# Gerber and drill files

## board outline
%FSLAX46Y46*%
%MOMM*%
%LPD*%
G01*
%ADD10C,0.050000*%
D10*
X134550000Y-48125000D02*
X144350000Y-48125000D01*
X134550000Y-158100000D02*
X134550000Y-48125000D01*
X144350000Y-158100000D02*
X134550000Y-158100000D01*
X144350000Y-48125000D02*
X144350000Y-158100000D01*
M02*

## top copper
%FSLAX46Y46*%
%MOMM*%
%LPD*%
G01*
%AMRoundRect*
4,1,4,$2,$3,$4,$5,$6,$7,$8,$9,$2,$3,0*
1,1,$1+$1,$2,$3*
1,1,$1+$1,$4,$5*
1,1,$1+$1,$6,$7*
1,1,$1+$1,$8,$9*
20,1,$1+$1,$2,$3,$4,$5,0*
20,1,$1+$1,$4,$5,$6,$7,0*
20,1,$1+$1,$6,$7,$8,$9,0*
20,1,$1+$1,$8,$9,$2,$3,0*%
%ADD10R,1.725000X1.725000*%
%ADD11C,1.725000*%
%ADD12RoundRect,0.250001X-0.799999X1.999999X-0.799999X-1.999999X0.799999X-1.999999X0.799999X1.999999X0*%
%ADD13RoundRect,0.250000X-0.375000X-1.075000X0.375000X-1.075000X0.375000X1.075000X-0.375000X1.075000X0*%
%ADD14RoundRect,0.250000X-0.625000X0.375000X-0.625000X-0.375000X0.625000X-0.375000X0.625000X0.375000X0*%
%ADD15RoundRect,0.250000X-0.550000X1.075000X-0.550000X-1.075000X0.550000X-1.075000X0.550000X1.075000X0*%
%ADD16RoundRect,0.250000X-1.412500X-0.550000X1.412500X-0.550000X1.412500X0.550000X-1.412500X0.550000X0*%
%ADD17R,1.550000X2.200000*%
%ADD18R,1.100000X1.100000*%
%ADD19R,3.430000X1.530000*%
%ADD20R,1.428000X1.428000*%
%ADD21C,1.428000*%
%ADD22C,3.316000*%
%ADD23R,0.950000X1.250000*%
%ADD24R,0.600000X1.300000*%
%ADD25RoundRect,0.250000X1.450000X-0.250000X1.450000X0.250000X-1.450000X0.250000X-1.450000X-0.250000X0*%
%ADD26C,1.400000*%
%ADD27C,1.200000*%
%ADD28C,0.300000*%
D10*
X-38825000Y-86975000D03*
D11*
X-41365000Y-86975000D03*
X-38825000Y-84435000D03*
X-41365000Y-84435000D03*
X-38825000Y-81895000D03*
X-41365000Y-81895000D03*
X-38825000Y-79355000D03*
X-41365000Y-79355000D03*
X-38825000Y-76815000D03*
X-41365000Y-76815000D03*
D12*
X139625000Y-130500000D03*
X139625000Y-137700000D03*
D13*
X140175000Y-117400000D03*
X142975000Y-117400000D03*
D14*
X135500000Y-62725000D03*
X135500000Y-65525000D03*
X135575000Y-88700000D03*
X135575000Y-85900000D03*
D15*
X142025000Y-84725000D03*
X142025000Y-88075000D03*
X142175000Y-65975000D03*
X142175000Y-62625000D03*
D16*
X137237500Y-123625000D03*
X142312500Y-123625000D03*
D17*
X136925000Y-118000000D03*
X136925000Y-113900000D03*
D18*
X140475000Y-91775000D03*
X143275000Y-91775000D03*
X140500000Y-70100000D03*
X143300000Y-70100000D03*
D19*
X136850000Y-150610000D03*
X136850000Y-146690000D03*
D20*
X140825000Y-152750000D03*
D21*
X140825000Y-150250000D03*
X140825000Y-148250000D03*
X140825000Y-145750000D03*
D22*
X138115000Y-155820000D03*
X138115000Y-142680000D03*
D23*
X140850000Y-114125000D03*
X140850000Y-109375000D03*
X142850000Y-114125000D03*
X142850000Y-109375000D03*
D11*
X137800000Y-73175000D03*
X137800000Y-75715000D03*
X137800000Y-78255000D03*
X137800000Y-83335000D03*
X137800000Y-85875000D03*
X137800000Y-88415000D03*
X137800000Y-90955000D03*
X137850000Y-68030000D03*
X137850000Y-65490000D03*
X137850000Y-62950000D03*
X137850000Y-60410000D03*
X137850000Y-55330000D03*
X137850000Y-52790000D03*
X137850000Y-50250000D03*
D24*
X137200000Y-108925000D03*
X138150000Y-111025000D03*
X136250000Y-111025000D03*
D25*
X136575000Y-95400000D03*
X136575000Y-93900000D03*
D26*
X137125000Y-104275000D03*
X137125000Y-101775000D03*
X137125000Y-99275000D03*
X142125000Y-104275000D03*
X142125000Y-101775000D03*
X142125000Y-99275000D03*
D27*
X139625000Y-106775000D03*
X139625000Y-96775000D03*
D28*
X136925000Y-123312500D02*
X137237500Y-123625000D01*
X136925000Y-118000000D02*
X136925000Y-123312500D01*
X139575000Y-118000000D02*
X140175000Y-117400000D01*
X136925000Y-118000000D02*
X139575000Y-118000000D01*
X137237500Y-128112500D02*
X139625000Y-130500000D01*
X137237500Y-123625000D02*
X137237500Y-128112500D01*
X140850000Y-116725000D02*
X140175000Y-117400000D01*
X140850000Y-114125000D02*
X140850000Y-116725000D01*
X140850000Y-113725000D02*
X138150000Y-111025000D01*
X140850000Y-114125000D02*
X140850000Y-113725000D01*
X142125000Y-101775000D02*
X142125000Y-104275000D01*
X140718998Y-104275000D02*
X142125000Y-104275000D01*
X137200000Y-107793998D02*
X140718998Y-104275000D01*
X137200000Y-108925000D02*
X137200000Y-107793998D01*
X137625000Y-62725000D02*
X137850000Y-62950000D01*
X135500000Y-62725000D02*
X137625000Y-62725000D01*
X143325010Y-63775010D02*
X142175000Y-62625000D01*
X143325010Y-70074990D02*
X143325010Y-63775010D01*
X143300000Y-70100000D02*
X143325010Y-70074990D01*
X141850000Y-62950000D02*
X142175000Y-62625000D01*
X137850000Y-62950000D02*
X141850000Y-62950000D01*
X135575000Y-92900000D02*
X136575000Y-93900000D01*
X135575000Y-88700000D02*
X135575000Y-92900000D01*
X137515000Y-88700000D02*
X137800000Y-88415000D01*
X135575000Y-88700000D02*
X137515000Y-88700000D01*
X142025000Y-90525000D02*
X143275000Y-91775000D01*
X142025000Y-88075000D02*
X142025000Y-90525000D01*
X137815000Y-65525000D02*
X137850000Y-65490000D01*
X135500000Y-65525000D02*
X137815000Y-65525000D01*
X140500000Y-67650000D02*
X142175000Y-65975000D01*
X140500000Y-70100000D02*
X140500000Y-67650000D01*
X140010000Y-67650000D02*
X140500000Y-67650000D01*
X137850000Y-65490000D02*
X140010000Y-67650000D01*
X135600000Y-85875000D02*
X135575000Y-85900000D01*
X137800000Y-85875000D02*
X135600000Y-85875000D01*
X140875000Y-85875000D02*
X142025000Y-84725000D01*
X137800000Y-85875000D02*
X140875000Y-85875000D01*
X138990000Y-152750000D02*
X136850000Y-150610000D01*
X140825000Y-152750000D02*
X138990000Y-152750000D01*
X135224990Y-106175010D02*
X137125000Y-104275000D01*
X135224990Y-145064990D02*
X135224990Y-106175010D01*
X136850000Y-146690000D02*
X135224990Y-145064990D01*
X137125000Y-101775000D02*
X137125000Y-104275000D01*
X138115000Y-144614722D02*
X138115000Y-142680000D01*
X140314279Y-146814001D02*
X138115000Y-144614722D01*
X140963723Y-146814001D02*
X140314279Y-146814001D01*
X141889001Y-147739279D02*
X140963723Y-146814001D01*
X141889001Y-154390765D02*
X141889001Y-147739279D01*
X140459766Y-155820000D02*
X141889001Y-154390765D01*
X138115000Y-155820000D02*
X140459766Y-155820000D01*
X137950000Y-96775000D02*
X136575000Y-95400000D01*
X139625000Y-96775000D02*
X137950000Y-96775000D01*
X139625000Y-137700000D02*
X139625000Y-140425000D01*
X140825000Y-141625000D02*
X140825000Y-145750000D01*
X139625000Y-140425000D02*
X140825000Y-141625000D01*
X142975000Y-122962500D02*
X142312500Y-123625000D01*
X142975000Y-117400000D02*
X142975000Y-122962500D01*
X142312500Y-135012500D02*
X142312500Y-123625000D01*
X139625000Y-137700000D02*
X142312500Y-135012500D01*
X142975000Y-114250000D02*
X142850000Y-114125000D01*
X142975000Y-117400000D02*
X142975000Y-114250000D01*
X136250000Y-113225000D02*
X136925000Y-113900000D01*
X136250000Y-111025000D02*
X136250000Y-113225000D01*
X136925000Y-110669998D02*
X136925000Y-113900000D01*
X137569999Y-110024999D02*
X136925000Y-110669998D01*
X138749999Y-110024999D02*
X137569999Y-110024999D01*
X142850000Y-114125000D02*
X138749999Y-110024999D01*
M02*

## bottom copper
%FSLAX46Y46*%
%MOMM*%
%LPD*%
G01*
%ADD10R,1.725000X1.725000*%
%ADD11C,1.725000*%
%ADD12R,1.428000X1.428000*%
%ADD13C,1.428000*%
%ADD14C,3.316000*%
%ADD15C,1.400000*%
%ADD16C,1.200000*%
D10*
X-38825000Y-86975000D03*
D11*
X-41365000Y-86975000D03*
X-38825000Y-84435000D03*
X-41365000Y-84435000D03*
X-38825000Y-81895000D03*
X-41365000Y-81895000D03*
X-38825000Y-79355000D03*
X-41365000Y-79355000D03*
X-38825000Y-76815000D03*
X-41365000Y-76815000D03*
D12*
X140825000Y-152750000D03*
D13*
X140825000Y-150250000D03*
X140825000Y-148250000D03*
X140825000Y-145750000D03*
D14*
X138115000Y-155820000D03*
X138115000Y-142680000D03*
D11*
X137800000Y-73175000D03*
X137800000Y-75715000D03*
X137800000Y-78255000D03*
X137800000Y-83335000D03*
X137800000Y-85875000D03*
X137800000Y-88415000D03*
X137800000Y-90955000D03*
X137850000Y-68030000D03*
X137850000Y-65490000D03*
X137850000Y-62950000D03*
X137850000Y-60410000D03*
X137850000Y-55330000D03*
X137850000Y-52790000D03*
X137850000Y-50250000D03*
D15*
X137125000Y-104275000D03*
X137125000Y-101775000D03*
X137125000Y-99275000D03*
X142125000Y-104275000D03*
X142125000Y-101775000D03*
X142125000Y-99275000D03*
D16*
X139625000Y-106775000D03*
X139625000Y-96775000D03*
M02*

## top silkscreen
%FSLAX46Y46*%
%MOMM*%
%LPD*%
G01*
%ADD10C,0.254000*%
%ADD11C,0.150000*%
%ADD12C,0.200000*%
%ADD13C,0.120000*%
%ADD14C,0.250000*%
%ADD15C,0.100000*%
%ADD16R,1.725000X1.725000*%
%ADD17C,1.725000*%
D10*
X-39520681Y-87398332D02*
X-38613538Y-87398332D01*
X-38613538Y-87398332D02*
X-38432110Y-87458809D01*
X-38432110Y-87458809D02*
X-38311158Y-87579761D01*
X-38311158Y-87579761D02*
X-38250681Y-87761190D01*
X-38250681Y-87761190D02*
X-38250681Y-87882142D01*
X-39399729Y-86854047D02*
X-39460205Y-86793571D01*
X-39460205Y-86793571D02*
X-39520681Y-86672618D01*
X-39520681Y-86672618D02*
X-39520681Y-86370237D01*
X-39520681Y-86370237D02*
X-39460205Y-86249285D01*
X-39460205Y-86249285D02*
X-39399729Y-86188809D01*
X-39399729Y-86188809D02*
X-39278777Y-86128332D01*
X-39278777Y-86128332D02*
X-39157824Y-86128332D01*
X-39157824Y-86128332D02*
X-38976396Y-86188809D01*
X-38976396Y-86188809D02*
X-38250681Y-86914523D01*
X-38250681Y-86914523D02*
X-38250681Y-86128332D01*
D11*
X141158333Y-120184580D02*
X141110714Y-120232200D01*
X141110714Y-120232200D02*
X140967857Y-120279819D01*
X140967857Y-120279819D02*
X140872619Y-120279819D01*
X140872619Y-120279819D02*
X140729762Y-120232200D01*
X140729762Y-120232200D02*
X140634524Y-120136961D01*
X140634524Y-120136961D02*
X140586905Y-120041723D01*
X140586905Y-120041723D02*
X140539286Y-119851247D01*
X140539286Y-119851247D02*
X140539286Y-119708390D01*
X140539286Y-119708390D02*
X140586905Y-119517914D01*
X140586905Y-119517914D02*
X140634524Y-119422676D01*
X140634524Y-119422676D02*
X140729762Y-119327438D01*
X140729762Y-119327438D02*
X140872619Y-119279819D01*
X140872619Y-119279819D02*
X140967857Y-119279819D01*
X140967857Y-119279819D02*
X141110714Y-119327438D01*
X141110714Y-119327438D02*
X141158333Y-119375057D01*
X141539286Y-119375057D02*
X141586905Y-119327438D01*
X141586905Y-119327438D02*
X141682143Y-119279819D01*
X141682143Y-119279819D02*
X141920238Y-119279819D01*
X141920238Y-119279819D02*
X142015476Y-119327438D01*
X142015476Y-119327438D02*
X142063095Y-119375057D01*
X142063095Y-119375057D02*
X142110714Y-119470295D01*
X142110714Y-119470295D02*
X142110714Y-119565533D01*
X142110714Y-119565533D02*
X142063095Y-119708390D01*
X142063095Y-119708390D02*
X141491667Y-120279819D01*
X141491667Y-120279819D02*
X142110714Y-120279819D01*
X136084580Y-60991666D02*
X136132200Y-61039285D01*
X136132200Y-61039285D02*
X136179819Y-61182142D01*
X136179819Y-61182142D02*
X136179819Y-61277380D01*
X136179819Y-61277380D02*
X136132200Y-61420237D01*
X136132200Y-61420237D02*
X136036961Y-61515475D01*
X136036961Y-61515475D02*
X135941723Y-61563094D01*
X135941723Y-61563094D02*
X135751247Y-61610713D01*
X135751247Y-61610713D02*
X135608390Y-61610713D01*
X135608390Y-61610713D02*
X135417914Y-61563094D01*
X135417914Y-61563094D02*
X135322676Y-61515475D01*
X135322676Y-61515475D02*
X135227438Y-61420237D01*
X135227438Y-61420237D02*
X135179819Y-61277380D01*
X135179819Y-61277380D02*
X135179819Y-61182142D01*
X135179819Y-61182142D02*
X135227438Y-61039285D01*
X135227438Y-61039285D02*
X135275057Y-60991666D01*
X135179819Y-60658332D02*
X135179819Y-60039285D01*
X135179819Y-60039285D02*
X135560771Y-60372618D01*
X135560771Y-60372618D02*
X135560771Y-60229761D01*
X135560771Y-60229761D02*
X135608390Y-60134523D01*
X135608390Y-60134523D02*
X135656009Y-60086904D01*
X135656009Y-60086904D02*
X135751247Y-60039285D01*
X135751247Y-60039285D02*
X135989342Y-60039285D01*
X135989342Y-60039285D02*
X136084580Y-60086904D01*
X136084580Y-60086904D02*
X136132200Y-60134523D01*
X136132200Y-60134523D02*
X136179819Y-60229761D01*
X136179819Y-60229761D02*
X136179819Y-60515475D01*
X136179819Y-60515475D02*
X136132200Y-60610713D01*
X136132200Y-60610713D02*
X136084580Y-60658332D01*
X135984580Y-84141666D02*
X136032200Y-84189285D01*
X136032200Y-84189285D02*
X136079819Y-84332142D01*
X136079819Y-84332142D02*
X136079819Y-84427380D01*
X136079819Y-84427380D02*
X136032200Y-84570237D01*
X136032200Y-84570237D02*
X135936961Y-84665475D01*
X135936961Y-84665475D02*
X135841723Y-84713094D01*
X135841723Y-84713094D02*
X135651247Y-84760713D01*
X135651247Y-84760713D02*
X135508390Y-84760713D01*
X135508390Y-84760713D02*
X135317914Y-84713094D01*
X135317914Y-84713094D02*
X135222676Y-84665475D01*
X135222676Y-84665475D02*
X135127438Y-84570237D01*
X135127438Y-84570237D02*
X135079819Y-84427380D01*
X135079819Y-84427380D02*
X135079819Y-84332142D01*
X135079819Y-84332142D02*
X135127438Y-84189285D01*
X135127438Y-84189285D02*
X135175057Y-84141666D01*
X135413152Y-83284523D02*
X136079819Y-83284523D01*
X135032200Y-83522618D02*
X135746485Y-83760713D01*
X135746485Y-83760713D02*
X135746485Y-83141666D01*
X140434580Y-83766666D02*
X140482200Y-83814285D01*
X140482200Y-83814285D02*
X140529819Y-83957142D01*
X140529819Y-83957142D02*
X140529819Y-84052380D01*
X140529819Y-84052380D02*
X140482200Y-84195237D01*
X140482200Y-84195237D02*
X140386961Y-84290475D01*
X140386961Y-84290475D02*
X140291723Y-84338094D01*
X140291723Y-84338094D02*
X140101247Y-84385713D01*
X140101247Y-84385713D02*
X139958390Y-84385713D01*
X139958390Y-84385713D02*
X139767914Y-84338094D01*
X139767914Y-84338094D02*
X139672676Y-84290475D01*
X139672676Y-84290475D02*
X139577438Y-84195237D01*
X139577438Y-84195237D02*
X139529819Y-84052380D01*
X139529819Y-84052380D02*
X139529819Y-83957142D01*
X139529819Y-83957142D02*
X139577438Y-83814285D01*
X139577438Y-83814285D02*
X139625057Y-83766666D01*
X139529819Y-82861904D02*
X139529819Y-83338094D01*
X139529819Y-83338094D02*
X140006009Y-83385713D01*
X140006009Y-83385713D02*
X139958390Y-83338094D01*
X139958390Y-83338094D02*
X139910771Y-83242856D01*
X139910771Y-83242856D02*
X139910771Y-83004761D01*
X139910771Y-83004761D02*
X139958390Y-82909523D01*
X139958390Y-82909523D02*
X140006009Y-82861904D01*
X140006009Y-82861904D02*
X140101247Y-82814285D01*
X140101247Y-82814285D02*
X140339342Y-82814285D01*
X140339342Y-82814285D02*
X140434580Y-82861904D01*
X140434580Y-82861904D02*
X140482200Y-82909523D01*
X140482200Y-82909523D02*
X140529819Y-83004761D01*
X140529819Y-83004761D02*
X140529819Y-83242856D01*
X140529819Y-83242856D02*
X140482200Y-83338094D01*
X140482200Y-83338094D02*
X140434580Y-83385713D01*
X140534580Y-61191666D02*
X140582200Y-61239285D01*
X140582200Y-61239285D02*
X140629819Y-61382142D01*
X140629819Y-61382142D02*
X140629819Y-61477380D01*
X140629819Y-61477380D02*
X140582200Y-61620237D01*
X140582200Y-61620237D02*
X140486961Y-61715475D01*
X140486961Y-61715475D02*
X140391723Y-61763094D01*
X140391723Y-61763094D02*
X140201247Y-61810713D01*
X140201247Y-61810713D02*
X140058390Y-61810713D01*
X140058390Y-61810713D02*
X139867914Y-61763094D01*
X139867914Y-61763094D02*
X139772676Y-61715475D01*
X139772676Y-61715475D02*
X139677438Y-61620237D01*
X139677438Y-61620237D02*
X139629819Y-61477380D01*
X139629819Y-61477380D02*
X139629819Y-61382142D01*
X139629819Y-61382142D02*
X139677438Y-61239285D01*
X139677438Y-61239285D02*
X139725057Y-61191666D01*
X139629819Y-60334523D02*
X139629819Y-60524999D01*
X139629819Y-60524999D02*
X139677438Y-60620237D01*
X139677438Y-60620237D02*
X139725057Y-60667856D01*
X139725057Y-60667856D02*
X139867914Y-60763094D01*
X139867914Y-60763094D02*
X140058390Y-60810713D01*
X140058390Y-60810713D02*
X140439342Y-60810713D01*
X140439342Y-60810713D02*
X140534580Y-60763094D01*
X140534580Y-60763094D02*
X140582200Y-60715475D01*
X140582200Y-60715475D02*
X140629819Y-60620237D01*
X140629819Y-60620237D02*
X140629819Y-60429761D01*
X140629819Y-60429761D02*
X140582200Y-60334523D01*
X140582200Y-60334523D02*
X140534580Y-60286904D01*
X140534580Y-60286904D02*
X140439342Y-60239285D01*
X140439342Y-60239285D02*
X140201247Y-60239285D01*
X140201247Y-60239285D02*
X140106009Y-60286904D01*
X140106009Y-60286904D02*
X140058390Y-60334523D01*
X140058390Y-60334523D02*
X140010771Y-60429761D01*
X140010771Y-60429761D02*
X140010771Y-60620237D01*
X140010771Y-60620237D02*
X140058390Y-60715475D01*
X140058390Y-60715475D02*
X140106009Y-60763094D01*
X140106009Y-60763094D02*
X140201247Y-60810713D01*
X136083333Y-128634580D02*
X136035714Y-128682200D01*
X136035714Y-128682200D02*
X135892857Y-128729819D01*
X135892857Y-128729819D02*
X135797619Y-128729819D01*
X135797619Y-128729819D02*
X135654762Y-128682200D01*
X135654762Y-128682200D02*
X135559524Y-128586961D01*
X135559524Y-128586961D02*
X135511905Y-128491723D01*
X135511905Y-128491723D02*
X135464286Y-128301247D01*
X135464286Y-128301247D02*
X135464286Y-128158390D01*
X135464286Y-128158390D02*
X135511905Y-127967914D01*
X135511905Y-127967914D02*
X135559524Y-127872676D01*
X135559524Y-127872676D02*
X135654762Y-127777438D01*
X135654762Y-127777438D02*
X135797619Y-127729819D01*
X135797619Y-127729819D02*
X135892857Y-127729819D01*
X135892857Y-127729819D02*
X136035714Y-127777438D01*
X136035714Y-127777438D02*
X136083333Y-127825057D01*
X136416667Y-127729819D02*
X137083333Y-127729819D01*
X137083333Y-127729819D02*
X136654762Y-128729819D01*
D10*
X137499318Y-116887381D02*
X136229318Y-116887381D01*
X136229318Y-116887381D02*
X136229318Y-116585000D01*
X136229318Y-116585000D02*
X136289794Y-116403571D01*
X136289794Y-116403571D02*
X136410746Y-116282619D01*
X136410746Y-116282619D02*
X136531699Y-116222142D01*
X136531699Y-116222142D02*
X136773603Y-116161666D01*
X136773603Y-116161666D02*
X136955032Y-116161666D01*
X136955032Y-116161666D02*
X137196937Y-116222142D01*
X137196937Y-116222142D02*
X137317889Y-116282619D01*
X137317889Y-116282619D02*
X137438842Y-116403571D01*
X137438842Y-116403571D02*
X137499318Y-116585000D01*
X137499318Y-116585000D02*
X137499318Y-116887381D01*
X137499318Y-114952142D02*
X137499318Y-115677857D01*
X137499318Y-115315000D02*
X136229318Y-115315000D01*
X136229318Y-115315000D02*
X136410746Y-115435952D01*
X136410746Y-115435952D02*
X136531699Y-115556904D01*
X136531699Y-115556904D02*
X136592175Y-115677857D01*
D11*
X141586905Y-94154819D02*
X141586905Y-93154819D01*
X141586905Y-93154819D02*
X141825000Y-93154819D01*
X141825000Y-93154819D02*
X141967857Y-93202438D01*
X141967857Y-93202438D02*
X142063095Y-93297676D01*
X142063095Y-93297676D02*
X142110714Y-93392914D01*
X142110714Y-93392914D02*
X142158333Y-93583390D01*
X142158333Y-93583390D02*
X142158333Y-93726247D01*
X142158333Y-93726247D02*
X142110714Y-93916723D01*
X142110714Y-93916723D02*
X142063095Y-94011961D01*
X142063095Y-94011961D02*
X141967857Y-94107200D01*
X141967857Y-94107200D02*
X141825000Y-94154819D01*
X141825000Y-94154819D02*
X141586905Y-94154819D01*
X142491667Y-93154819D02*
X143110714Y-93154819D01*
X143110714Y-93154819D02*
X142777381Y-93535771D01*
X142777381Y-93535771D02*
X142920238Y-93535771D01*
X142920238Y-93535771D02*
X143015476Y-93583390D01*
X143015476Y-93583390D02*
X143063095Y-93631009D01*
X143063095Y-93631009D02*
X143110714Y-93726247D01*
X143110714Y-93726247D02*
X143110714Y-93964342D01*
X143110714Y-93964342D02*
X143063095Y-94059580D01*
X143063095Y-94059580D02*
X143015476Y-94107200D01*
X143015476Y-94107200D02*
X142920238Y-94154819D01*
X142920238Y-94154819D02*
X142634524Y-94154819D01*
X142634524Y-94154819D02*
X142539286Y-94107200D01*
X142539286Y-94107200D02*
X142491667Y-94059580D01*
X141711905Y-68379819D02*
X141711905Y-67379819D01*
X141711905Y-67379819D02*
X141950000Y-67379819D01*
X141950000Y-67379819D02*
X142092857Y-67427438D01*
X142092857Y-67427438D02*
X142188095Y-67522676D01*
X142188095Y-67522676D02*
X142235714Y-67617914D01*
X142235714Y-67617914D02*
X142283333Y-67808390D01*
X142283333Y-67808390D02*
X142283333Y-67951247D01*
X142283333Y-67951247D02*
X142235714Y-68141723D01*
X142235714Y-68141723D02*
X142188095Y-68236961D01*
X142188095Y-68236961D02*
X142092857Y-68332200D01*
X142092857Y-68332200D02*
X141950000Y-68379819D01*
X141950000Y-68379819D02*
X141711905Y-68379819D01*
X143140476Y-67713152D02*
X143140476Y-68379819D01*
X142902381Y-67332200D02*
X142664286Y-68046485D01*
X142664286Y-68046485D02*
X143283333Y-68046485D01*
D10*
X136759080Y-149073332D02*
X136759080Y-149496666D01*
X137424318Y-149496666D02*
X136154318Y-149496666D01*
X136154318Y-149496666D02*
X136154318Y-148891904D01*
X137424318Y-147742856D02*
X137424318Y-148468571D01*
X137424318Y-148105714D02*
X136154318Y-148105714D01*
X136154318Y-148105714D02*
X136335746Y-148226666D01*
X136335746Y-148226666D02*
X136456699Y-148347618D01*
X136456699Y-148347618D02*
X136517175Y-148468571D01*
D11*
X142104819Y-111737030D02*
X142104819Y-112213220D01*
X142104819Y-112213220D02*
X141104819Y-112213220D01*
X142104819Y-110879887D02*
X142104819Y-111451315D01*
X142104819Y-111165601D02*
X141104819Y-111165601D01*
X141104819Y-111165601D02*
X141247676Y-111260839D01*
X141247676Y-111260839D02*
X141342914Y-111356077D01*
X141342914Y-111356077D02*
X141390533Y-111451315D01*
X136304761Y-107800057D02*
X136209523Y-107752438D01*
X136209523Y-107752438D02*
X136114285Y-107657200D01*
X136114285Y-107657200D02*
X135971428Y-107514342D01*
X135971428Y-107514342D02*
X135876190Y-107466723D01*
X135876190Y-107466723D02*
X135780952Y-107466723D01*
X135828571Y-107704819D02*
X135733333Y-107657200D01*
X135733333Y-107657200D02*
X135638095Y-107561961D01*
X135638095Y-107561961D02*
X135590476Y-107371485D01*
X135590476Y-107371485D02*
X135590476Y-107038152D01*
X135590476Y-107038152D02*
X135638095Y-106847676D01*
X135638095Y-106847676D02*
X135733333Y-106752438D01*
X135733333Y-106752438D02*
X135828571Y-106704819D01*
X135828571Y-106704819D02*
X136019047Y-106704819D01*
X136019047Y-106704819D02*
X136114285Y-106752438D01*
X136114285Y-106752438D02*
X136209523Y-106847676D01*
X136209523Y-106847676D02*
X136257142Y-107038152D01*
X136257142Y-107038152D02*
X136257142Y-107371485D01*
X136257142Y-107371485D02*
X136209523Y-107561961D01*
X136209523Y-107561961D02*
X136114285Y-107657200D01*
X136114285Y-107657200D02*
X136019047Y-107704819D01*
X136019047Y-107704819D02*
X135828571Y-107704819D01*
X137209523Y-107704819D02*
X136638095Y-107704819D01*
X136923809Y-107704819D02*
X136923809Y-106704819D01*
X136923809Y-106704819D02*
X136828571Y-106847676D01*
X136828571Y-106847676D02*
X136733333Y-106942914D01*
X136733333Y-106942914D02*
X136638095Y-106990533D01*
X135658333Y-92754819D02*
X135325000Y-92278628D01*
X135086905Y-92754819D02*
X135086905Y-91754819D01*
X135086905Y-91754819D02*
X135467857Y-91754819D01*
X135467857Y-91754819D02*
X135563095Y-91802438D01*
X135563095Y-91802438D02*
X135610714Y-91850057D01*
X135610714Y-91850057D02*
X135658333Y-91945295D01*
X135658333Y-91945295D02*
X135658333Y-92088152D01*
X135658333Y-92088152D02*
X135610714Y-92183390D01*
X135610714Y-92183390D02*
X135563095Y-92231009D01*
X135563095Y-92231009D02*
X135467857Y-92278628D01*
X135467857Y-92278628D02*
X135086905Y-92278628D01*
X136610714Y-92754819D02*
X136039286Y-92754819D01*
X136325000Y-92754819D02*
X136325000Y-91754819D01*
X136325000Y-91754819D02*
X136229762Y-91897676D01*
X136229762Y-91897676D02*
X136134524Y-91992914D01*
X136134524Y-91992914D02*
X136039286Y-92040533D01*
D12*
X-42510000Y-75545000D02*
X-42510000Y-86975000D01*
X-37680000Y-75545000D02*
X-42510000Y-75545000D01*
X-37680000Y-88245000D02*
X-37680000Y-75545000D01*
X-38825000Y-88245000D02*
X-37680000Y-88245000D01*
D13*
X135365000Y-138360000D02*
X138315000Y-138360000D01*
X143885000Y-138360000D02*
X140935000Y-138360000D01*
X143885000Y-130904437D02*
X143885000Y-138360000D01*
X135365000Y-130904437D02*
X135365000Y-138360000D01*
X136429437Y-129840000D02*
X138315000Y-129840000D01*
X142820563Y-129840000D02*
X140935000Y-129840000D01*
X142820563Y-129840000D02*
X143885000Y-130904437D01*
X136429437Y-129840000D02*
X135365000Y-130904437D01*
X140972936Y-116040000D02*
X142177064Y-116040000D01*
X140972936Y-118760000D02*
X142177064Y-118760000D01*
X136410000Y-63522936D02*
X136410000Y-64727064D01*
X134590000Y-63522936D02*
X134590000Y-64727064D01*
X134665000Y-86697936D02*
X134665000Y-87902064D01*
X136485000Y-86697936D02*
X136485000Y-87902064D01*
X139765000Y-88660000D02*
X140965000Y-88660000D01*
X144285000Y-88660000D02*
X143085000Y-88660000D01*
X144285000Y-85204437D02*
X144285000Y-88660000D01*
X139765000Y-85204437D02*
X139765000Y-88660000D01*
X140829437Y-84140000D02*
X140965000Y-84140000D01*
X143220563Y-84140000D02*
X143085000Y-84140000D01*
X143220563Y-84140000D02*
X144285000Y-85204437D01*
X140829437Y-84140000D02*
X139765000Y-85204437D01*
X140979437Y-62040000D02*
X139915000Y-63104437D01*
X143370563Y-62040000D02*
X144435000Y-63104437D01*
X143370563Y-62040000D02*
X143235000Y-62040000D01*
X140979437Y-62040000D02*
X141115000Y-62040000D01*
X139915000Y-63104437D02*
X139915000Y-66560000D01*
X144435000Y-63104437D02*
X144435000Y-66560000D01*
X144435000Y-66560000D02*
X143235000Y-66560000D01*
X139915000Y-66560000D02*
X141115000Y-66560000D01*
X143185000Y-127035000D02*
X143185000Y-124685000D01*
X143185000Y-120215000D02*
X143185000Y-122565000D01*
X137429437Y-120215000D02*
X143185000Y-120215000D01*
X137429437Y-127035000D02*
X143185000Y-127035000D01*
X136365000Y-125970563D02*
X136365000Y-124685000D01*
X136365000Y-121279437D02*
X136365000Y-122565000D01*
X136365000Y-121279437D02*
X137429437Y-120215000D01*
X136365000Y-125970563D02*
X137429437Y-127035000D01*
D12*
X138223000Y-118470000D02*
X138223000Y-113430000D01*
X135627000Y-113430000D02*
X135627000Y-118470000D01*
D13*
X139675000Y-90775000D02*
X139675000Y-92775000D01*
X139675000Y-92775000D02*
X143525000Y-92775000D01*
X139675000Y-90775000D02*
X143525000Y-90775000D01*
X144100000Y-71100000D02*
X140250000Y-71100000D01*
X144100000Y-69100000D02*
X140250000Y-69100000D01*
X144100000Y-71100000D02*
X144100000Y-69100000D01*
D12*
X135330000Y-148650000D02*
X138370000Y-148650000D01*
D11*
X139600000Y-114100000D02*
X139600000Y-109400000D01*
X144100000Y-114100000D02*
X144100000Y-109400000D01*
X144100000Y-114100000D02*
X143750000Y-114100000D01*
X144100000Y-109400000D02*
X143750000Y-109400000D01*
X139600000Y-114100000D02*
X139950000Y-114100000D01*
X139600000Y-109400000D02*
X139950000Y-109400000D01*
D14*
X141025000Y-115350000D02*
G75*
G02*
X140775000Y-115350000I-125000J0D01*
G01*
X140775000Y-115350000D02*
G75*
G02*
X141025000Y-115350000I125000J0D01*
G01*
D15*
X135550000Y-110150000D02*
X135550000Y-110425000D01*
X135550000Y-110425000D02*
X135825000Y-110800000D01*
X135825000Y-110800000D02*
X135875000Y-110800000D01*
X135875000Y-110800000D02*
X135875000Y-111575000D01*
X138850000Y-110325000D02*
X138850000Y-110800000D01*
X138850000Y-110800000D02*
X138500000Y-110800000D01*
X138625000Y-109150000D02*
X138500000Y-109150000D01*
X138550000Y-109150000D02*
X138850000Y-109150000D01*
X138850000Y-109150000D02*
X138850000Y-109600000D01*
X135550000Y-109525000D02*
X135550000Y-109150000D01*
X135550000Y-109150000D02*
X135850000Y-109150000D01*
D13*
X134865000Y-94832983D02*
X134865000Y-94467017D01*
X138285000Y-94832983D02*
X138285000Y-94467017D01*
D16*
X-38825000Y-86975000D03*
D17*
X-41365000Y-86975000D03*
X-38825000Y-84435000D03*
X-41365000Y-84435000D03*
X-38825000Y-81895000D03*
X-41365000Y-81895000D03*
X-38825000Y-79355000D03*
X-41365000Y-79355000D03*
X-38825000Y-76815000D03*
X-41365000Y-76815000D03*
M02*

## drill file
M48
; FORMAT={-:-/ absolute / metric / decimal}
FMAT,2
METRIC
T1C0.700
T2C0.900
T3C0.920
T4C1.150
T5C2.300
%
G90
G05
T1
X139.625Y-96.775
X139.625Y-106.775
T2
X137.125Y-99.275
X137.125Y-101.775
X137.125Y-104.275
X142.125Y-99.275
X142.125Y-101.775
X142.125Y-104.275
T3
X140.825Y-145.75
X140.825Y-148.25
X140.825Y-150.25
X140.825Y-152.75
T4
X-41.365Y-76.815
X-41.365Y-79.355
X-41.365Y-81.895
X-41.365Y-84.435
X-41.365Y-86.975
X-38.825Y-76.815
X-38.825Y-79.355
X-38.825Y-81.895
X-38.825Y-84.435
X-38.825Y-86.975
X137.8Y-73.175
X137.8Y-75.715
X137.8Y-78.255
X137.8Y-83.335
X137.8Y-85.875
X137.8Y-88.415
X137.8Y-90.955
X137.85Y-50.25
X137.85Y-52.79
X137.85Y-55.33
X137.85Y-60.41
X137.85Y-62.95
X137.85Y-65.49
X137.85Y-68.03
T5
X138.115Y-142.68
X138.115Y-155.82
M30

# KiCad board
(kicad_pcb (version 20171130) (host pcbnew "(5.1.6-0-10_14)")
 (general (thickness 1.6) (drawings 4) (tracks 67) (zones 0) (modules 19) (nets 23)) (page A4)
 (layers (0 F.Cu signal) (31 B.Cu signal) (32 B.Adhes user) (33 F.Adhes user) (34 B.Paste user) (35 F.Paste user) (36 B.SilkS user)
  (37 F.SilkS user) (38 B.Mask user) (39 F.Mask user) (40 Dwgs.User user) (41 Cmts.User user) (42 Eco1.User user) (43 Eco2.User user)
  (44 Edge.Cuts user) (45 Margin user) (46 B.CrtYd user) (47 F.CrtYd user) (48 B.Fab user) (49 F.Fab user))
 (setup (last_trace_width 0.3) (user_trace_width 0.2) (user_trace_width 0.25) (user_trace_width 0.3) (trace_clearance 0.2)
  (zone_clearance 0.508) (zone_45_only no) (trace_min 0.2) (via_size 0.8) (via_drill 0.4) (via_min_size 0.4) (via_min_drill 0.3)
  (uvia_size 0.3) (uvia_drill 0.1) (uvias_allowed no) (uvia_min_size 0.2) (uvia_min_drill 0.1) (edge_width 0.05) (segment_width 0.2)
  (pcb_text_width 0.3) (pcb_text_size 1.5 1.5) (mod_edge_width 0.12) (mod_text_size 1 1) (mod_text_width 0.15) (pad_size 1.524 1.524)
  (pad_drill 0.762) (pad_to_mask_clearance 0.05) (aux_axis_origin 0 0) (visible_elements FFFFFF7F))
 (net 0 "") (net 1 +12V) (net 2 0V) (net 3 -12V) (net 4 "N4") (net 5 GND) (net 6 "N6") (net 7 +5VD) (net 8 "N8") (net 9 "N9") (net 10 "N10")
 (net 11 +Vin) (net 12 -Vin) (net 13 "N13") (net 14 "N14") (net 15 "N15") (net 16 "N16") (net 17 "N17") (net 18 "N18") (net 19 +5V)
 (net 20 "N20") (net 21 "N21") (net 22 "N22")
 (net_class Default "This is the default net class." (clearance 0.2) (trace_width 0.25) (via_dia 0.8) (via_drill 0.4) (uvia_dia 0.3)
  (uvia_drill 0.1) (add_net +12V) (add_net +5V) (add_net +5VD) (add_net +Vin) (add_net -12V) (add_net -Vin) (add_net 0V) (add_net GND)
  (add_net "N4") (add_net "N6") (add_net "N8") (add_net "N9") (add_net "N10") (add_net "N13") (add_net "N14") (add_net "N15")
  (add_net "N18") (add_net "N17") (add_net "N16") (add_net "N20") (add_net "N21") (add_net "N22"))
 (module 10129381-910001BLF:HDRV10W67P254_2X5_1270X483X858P (layer F.Cu) (at -38.825 86.975 90)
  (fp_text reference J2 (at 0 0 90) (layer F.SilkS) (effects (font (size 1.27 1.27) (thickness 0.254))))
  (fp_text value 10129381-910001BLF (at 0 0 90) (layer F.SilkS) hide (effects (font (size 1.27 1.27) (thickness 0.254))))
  (fp_line (start 11.43 -3.685) (end 0 -3.685) (layer F.SilkS) (width 0.2))
  (fp_line (start 11.43 1.145) (end 11.43 -3.685) (layer F.SilkS) (width 0.2))
  (fp_line (start -1.27 1.145) (end 11.43 1.145) (layer F.SilkS) (width 0.2))
  (fp_line (start -1.27 0) (end -1.27 1.145) (layer F.SilkS) (width 0.2))
  (pad 1 thru_hole rect (at 0 0 180) (size 1.725 1.725) (drill 1.15) (layers *.Cu *.Mask F.SilkS) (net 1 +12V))
  (pad 2 thru_hole circle (at 0 -2.54 180) (size 1.725 1.725) (drill 1.15) (layers *.Cu *.Mask F.SilkS) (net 1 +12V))
  (pad 3 thru_hole circle (at 2.54 0 180) (size 1.725 1.725) (drill 1.15) (layers *.Cu *.Mask F.SilkS) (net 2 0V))
  (pad 4 thru_hole circle (at 2.54 -2.54 180) (size 1.725 1.725) (drill 1.15) (layers *.Cu *.Mask F.SilkS) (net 2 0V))
  (pad 5 thru_hole circle (at 5.08 0 180) (size 1.725 1.725) (drill 1.15) (layers *.Cu *.Mask F.SilkS) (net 2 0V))
  (pad 6 thru_hole circle (at 5.08 -2.54 180) (size 1.725 1.725) (drill 1.15) (layers *.Cu *.Mask F.SilkS) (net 2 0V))
  (pad 7 thru_hole circle (at 7.62 0 180) (size 1.725 1.725) (drill 1.15) (layers *.Cu *.Mask F.SilkS) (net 2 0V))
  (pad 8 thru_hole circle (at 7.62 -2.54 180) (size 1.725 1.725) (drill 1.15) (layers *.Cu *.Mask F.SilkS) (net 2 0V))
  (pad 9 thru_hole circle (at 10.16 0 180) (size 1.725 1.725) (drill 1.15) (layers *.Cu *.Mask F.SilkS) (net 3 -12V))
  (pad 10 thru_hole circle (at 10.16 -2.54 180) (size 1.725 1.725) (drill 1.15) (layers *.Cu *.Mask F.SilkS) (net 3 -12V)))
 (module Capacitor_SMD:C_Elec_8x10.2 (layer F.Cu) (at 139.625 134.1 270)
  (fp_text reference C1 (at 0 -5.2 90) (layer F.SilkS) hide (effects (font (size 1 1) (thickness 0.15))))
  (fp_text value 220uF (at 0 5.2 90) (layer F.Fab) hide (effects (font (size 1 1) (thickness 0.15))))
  (fp_line (start 4.26 4.26) (end 4.26 1.31) (layer F.SilkS) (width 0.12))
  (fp_line (start 4.26 -4.26) (end 4.26 -1.31) (layer F.SilkS) (width 0.12))
  (fp_line (start -3.195563 -4.26) (end 4.26 -4.26) (layer F.SilkS) (width 0.12))
  (fp_line (start -3.195563 4.26) (end 4.26 4.26) (layer F.SilkS) (width 0.12))
  (fp_line (start -4.26 3.195563) (end -4.26 1.31) (layer F.SilkS) (width 0.12))
  (fp_line (start -4.26 -3.195563) (end -4.26 -1.31) (layer F.SilkS) (width 0.12))
  (fp_line (start -4.26 -3.195563) (end -3.195563 -4.26) (layer F.SilkS) (width 0.12))
  (fp_line (start -4.26 3.195563) (end -3.195563 4.26) (layer F.SilkS) (width 0.12))
  (pad 1 smd roundrect (at -3.6 0 270) (size 4.5 2.1) (layers F.Cu F.Paste F.Mask) (roundrect_rratio 0.119048) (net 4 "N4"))
  (pad 2 smd roundrect (at 3.6 0 270) (size 4.5 2.1) (layers F.Cu F.Paste F.Mask) (roundrect_rratio 0.119048) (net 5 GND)))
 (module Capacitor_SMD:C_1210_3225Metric (layer F.Cu) (at 141.575 117.4)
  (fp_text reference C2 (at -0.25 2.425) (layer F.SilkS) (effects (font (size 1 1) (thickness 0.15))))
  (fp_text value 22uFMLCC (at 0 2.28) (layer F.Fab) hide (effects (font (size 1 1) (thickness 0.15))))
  (fp_line (start -0.602064 -1.36) (end 0.602064 -1.36) (layer F.SilkS) (width 0.12))
  (fp_line (start -0.602064 1.36) (end 0.602064 1.36) (layer F.SilkS) (width 0.12))
  (pad 1 smd roundrect (at -1.4 0) (size 1.25 2.65) (layers F.Cu F.Paste F.Mask) (roundrect_rratio 0.2) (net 4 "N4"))
  (pad 2 smd roundrect (at 1.4 0) (size 1.25 2.65) (layers F.Cu F.Paste F.Mask) (roundrect_rratio 0.2) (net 5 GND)))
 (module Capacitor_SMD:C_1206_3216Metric (layer F.Cu) (at 135.5 64.125 270)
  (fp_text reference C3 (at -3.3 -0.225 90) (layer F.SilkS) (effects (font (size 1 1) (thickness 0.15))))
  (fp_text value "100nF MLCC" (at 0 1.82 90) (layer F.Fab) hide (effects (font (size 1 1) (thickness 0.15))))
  (fp_line (start -0.602064 -0.91) (end 0.602064 -0.91) (layer F.SilkS) (width 0.12))
  (fp_line (start -0.602064 0.91) (end 0.602064 0.91) (layer F.SilkS) (width 0.12))
  (pad 1 smd roundrect (at -1.4 0 270) (size 1.25 1.75) (layers F.Cu F.Paste F.Mask) (roundrect_rratio 0.2) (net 2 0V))
  (pad 2 smd roundrect (at 1.4 0 270) (size 1.25 1.75) (layers F.Cu F.Paste F.Mask) (roundrect_rratio 0.2) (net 3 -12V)))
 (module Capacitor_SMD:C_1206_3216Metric (layer F.Cu) (at 135.575 87.3 270)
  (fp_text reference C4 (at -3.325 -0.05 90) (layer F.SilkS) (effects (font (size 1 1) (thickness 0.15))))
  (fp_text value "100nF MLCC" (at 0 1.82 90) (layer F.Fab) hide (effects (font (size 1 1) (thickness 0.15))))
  (fp_line (start -0.602064 0.91) (end 0.602064 0.91) (layer F.SilkS) (width 0.12))
  (fp_line (start -0.602064 -0.91) (end 0.602064 -0.91) (layer F.SilkS) (width 0.12))
  (pad 2 smd roundrect (at 1.4 0 270) (size 1.25 1.75) (layers F.Cu F.Paste F.Mask) (roundrect_rratio 0.2) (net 2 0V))
  (pad 1 smd roundrect (at -1.4 0 270) (size 1.25 1.75) (layers F.Cu F.Paste F.Mask) (roundrect_rratio 0.2) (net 1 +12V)))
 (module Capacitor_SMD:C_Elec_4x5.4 (layer F.Cu) (at 142.025 86.4 270)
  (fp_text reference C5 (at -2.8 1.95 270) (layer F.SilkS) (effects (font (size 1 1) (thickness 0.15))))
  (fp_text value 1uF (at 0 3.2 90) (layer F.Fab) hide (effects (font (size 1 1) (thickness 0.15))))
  (fp_line (start 2.26 2.26) (end 2.26 1.06) (layer F.SilkS) (width 0.12))
  (fp_line (start 2.26 -2.26) (end 2.26 -1.06) (layer F.SilkS) (width 0.12))
  (fp_line (start -1.195563 -2.26) (end 2.26 -2.26) (layer F.SilkS) (width 0.12))
  (fp_line (start -1.195563 2.26) (end 2.26 2.26) (layer F.SilkS) (width 0.12))
  (fp_line (start -2.26 1.195563) (end -2.26 1.06) (layer F.SilkS) (width 0.12))
  (fp_line (start -2.26 -1.195563) (end -2.26 -1.06) (layer F.SilkS) (width 0.12))
  (fp_line (start -2.26 -1.195563) (end -1.195563 -2.26) (layer F.SilkS) (width 0.12))
  (fp_line (start -2.26 1.195563) (end -1.195563 2.26) (layer F.SilkS) (width 0.12))
  (pad 1 smd roundrect (at -1.675 0 270) (size 2.65 1.6) (layers F.Cu F.Paste F.Mask) (roundrect_rratio 0.15625) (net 1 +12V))
  (pad 2 smd roundrect (at 1.675 0 270) (size 2.65 1.6) (layers F.Cu F.Paste F.Mask) (roundrect_rratio 0.15625) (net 2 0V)))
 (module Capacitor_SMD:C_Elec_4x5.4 (layer F.Cu) (at 142.175 64.3 270)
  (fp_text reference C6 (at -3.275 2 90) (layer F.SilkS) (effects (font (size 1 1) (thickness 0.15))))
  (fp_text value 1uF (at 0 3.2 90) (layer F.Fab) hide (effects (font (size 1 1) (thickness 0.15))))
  (fp_line (start -2.26 1.195563) (end -1.195563 2.26) (layer F.SilkS) (width 0.12))
  (fp_line (start -2.26 -1.195563) (end -1.195563 -2.26) (layer F.SilkS) (width 0.12))
  (fp_line (start -2.26 -1.195563) (end -2.26 -1.06) (layer F.SilkS) (width 0.12))
  (fp_line (start -2.26 1.195563) (end -2.26 1.06) (layer F.SilkS) (width 0.12))
  (fp_line (start -1.195563 2.26) (end 2.26 2.26) (layer F.SilkS) (width 0.12))
  (fp_line (start -1.195563 -2.26) (end 2.26 -2.26) (layer F.SilkS) (width 0.12))
  (fp_line (start 2.26 -2.26) (end 2.26 -1.06) (layer F.SilkS) (width 0.12))
  (fp_line (start 2.26 2.26) (end 2.26 1.06) (layer F.SilkS) (width 0.12))
  (pad 2 smd roundrect (at 1.675 0 270) (size 2.65 1.6) (layers F.Cu F.Paste F.Mask) (roundrect_rratio 0.15625) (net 3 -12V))
  (pad 1 smd roundrect (at -1.675 0 270) (size 2.65 1.6) (layers F.Cu F.Paste F.Mask) (roundrect_rratio 0.15625) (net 2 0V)))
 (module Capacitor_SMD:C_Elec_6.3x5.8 (layer F.Cu) (at 139.775 123.625)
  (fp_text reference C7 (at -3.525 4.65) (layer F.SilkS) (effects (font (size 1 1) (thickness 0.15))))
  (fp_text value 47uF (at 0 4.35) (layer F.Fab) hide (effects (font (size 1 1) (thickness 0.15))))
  (fp_line (start 3.41 3.41) (end 3.41 1.06) (layer F.SilkS) (width 0.12))
  (fp_line (start 3.41 -3.41) (end 3.41 -1.06) (layer F.SilkS) (width 0.12))
  (fp_line (start -2.345563 -3.41) (end 3.41 -3.41) (layer F.SilkS) (width 0.12))
  (fp_line (start -2.345563 3.41) (end 3.41 3.41) (layer F.SilkS) (width 0.12))
  (fp_line (start -3.41 2.345563) (end -3.41 1.06) (layer F.SilkS) (width 0.12))
  (fp_line (start -3.41 -2.345563) (end -3.41 -1.06) (layer F.SilkS) (width 0.12))
  (fp_line (start -3.41 -2.345563) (end -2.345563 -3.41) (layer F.SilkS) (width 0.12))
  (fp_line (start -3.41 2.345563) (end -2.345563 3.41) (layer F.SilkS) (width 0.12))
  (pad 1 smd roundrect (at -2.5375 0) (size 3.325 1.6) (layers F.Cu F.Paste F.Mask) (roundrect_rratio 0.15625) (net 4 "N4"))
  (pad 2 smd roundrect (at 2.5375 0) (size 3.325 1.6) (layers F.Cu F.Paste F.Mask) (roundrect_rratio 0.15625) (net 5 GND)))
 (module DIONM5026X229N (layer F.Cu) (at 136.925 115.95 90)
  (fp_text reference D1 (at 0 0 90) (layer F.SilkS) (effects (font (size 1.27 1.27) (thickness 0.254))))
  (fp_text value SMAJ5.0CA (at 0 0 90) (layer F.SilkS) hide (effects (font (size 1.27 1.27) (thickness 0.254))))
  (fp_line (start -2.52 1.298) (end 2.52 1.298) (layer F.SilkS) (width 0.2))
  (fp_line (start 2.52 -1.298) (end -2.52 -1.298) (layer F.SilkS) (width 0.2))
  (pad 1 smd rect (at -2.05 0 180) (size 1.55 2.2) (layers F.Cu F.Paste F.Mask) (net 4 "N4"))
  (pad 2 smd rect (at 2.05 0 180) (size 1.55 2.2) (layers F.Cu F.Paste F.Mask) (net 5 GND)))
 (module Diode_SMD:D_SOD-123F (layer F.Cu) (at 141.875 91.775)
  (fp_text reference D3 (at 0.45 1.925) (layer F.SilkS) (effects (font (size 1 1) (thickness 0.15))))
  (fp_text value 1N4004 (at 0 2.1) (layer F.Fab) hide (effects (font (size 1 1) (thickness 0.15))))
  (fp_line (start -2.2 -1) (end -2.2 1) (layer F.SilkS) (width 0.12))
  (fp_line (start -2.2 1) (end 1.65 1) (layer F.SilkS) (width 0.12))
  (fp_line (start -2.2 -1) (end 1.65 -1) (layer F.SilkS) (width 0.12))
  (pad 1 smd rect (at -1.4 0) (size 1.1 1.1) (layers F.Cu F.Paste F.Mask) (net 1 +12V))
  (pad 2 smd rect (at 1.4 0) (size 1.1 1.1) (layers F.Cu F.Paste F.Mask) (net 2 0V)))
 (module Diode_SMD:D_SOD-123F (layer F.Cu) (at 141.9 70.1 180)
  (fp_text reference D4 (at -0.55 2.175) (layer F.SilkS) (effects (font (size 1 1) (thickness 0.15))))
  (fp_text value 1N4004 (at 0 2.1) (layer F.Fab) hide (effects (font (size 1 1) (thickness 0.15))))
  (fp_line (start -2.2 -1) (end 1.65 -1) (layer F.SilkS) (width 0.12))
  (fp_line (start -2.2 1) (end 1.65 1) (layer F.SilkS) (width 0.12))
  (fp_line (start -2.2 -1) (end -2.2 1) (layer F.SilkS) (width 0.12))
  (pad 2 smd rect (at 1.4 0 180) (size 1.1 1.1) (layers F.Cu F.Paste F.Mask) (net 3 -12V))
  (pad 1 smd rect (at -1.4 0 180) (size 1.1 1.1) (layers F.Cu F.Paste F.Mask) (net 2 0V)))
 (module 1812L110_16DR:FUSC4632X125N (layer F.Cu) (at 136.85 148.65 90)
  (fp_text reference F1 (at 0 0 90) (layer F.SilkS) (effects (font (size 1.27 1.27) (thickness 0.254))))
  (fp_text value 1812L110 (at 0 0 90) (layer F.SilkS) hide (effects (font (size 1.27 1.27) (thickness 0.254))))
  (fp_line (start 0 -1.52) (end 0 1.52) (layer F.SilkS) (width 0.2))
  (pad 1 smd rect (at -1.96 0 90) (size 1.53 3.43) (layers F.Cu F.Paste F.Mask) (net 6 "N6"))
  (pad 2 smd rect (at 1.96 0 90) (size 1.53 3.43) (layers F.Cu F.Paste F.Mask) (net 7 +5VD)))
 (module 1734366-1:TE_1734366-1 (layer B.Cu) (at 140.825 152.75 90)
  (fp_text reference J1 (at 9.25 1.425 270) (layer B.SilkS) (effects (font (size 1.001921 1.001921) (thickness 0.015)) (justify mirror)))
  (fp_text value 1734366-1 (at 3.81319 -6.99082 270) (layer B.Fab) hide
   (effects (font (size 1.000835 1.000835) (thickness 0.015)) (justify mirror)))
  (pad 1 thru_hole rect (at 0 0 90) (size 1.428 1.428) (drill 0.92) (layers *.Cu *.Mask) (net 6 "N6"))
  (pad 2 thru_hole circle (at 2.5 0 90) (size 1.428 1.428) (drill 0.92) (layers *.Cu *.Mask) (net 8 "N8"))
  (pad 3 thru_hole circle (at 4.5 0 90) (size 1.428 1.428) (drill 0.92) (layers *.Cu *.Mask) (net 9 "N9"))
  (pad 4 thru_hole circle (at 7 0 90) (size 1.428 1.428) (drill 0.92) (layers *.Cu *.Mask) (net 5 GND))
  (pad SH1 thru_hole circle (at -3.07 -2.71 90) (size 3.316 3.316) (drill 2.3) (layers *.Cu *.Mask) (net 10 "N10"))
  (pad SH2 thru_hole circle (at 10.07 -2.71 90) (size 3.316 3.316) (drill 2.3) (layers *.Cu *.Mask) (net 10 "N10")))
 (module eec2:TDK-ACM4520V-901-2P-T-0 (layer F.Cu) (at 141.85 111.75 90)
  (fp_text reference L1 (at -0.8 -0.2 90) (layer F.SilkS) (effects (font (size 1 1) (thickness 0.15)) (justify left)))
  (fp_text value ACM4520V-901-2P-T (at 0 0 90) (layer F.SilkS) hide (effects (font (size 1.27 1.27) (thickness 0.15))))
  (fp_line (start -2.35 -2.25) (end 2.35 -2.25) (layer F.SilkS) (width 0.15))
  (fp_line (start -2.35 2.25) (end 2.35 2.25) (layer F.SilkS) (width 0.15))
  (fp_line (start -2.35 2.25) (end -2.35 1.9) (layer F.SilkS) (width 0.15))
  (fp_line (start 2.35 2.25) (end 2.35 1.9) (layer F.SilkS) (width 0.15))
  (fp_line (start -2.35 -2.25) (end -2.35 -1.9) (layer F.SilkS) (width 0.15))
  (fp_line (start 2.35 -2.25) (end 2.35 -1.9) (layer F.SilkS) (width 0.15))
  (fp_circle (center -3.6 -0.95) (end -3.475 -0.95) (layer F.SilkS) (width 0.25))
  (pad 1 smd rect (at -2.375 -1 90) (size 1.25 0.95) (layers F.Cu F.Paste F.Mask) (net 4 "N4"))
  (pad 4 smd rect (at 2.375 -1 90) (size 1.25 0.95) (layers F.Cu F.Paste F.Mask) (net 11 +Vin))
  (pad 2 smd rect (at -2.375 1 90) (size 1.25 0.95) (layers F.Cu F.Paste F.Mask) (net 5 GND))
  (pad 3 smd rect (at 2.375 1 90) (size 1.25 0.95) (layers F.Cu F.Paste F.Mask) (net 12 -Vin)))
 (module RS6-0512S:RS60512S (layer B.Cu) (at 137.8 73.175 270)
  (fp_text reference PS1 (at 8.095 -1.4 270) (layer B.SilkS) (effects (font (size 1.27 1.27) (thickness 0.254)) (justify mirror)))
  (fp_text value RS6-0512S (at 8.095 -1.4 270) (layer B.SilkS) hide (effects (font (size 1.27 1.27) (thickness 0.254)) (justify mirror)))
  (pad 1 thru_hole circle (at 0 0 180) (size 1.725 1.725) (drill 1.15) (layers *.Cu *.Mask B.SilkS) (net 12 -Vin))
  (pad 2 thru_hole circle (at 2.54 0 180) (size 1.725 1.725) (drill 1.15) (layers *.Cu *.Mask B.SilkS) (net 11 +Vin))
  (pad 3 thru_hole circle (at 5.08 0 180) (size 1.725 1.725) (drill 1.15) (layers *.Cu *.Mask B.SilkS) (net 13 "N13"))
  (pad 5 thru_hole circle (at 10.16 0 180) (size 1.725 1.725) (drill 1.15) (layers *.Cu *.Mask B.SilkS) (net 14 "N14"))
  (pad 6 thru_hole circle (at 12.7 0 180) (size 1.725 1.725) (drill 1.15) (layers *.Cu *.Mask B.SilkS) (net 1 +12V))
  (pad 7 thru_hole circle (at 15.24 0 180) (size 1.725 1.725) (drill 1.15) (layers *.Cu *.Mask B.SilkS) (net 2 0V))
  (pad 8 thru_hole circle (at 17.78 0 180) (size 1.725 1.725) (drill 1.15) (layers *.Cu *.Mask B.SilkS) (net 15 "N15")))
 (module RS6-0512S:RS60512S (layer B.Cu) (at 137.85 50.25 270)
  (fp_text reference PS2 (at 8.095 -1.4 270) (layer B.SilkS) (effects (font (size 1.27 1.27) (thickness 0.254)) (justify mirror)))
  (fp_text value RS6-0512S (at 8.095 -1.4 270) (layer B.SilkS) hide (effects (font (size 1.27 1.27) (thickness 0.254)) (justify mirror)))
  (pad 8 thru_hole circle (at 17.78 0 180) (size 1.725 1.725) (drill 1.15) (layers *.Cu *.Mask B.SilkS) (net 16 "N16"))
  (pad 7 thru_hole circle (at 15.24 0 180) (size 1.725 1.725) (drill 1.15) (layers *.Cu *.Mask B.SilkS) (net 3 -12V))
  (pad 6 thru_hole circle (at 12.7 0 180) (size 1.725 1.725) (drill 1.15) (layers *.Cu *.Mask B.SilkS) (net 2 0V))
  (pad 5 thru_hole circle (at 10.16 0 180) (size 1.725 1.725) (drill 1.15) (layers *.Cu *.Mask B.SilkS) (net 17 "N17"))
  (pad 3 thru_hole circle (at 5.08 0 180) (size 1.725 1.725) (drill 1.15) (layers *.Cu *.Mask B.SilkS) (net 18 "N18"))
  (pad 2 thru_hole circle (at 2.54 0 180) (size 1.725 1.725) (drill 1.15) (layers *.Cu *.Mask B.SilkS) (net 11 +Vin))
  (pad 1 thru_hole circle (at 0 0 180) (size 1.725 1.725) (drill 1.15) (layers *.Cu *.Mask B.SilkS) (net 12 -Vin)))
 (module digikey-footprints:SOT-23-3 (layer F.Cu) (at 137.2 109.975 90)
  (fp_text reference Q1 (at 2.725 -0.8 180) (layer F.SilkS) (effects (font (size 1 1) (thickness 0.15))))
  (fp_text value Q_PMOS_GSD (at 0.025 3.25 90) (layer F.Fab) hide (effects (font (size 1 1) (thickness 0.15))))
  (fp_line (start -0.175 -1.65) (end -0.45 -1.65) (layer F.SilkS) (width 0.1))
  (fp_line (start -0.45 -1.65) (end -0.825 -1.375) (layer F.SilkS) (width 0.1))
  (fp_line (start -0.825 -1.375) (end -0.825 -1.325) (layer F.SilkS) (width 0.1))
  (fp_line (start -0.825 -1.325) (end -1.6 -1.325) (layer F.SilkS) (width 0.1))
  (fp_line (start -0.35 1.65) (end -0.825 1.65) (layer F.SilkS) (width 0.1))
  (fp_line (start -0.825 1.65) (end -0.825 1.3) (layer F.SilkS) (width 0.1))
  (fp_line (start 0.825 1.425) (end 0.825 1.3) (layer F.SilkS) (width 0.1))
  (fp_line (start 0.825 1.35) (end 0.825 1.65) (layer F.SilkS) (width 0.1))
  (fp_line (start 0.825 1.65) (end 0.375 1.65) (layer F.SilkS) (width 0.1))
  (fp_line (start 0.45 -1.65) (end 0.825 -1.65) (layer F.SilkS) (width 0.1))
  (fp_line (start 0.825 -1.65) (end 0.825 -1.35) (layer F.SilkS) (width 0.1))
  (pad 3 smd rect (at 1.05 0 90) (size 1.3 0.6) (layers F.Cu F.Paste F.Mask) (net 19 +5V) (solder_mask_margin 0.07))
  (pad 2 smd rect (at -1.05 0.95 90) (size 1.3 0.6) (layers F.Cu F.Paste F.Mask) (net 4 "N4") (solder_mask_margin 0.07))
  (pad 1 smd rect (at -1.05 -0.95 90) (size 1.3 0.6) (layers F.Cu F.Paste F.Mask) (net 5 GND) (solder_mask_margin 0.07)))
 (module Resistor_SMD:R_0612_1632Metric (layer F.Cu) (at 136.575 94.65 90)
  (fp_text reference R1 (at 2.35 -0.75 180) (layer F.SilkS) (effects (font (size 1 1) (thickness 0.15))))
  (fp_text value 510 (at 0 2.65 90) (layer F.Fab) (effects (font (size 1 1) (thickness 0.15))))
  (fp_line (start -0.182983 -1.71) (end 0.182983 -1.71) (layer F.SilkS) (width 0.12))
  (fp_line (start -0.182983 1.71) (end 0.182983 1.71) (layer F.SilkS) (width 0.12))
  (pad 1 smd roundrect (at -0.75 0 90) (size 1 3.4) (layers F.Cu F.Paste F.Mask) (roundrect_rratio 0.25) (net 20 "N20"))
  (pad 2 smd roundrect (at 0.75 0 90) (size 1 3.4) (layers F.Cu F.Paste F.Mask) (roundrect_rratio 0.25) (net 2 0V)))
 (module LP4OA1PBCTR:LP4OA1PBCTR (layer B.Cu) (at 137.125 104.275 270)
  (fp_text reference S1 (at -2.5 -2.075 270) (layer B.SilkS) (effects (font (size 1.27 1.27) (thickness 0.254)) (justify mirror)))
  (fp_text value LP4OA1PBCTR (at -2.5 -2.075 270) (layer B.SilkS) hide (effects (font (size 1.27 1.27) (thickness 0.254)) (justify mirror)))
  (pad 1 thru_hole circle (at 0 0 180) (size 1.4 1.4) (drill 0.9) (layers *.Cu *.Mask B.SilkS) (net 7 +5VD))
  (pad 2 thru_hole circle (at -2.5 0 180) (size 1.4 1.4) (drill 0.9) (layers *.Cu *.Mask B.SilkS) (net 7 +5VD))
  (pad 3 thru_hole circle (at -5 0 180) (size 1.4 1.4) (drill 0.9) (layers *.Cu *.Mask B.SilkS) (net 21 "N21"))
  (pad 4 thru_hole circle (at 0 -5 180) (size 1.4 1.4) (drill 0.9) (layers *.Cu *.Mask B.SilkS) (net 19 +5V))
  (pad 5 thru_hole circle (at -2.5 -5 180) (size 1.4 1.4) (drill 0.9) (layers *.Cu *.Mask B.SilkS) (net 19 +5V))
  (pad 6 thru_hole circle (at -5 -5 180) (size 1.4 1.4) (drill 0.9) (layers *.Cu *.Mask B.SilkS) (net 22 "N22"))
  (pad L1 thru_hole circle (at 2.5 -2.5 180) (size 1.2 1.2) (drill 0.7) (layers *.Cu *.Mask B.SilkS) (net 1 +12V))
  (pad L2 thru_hole circle (at -7.5 -2.5 180) (size 1.2 1.2) (drill 0.7) (layers *.Cu *.Mask B.SilkS) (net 20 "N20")))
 (gr_line (start 134.55 48.125) (end 144.35 48.125) (layer Edge.Cuts) (width 0.05))
 (gr_line (start 134.55 158.1) (end 134.55 48.125) (layer Edge.Cuts) (width 0.05))
 (gr_line (start 144.35 158.1) (end 134.55 158.1) (layer Edge.Cuts) (width 0.05))
 (gr_line (start 144.35 48.125) (end 144.35 158.1) (layer Edge.Cuts) (width 0.05))
 (segment (start 136.925 123.3125) (end 137.2375 123.625) (width 0.3) (layer F.Cu) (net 4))
 (segment (start 136.925 118) (end 136.925 123.3125) (width 0.3) (layer F.Cu) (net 4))
 (segment (start 139.575 118) (end 140.175 117.4) (width 0.3) (layer F.Cu) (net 4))
 (segment (start 136.925 118) (end 139.575 118) (width 0.3) (layer F.Cu) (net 4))
 (segment (start 137.2375 128.1125) (end 139.625 130.5) (width 0.3) (layer F.Cu) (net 4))
 (segment (start 137.2375 123.625) (end 137.2375 128.1125) (width 0.3) (layer F.Cu) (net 4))
 (segment (start 140.85 116.725) (end 140.175 117.4) (width 0.3) (layer F.Cu) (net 4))
 (segment (start 140.85 114.125) (end 140.85 116.725) (width 0.3) (layer F.Cu) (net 4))
 (segment (start 140.85 113.725) (end 138.15 111.025) (width 0.3) (layer F.Cu) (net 4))
 (segment (start 140.85 114.125) (end 140.85 113.725) (width 0.3) (layer F.Cu) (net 4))
 (segment (start 142.125 101.775) (end 142.125 104.275) (width 0.3) (layer F.Cu) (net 19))
 (segment (start 140.718998 104.275) (end 142.125 104.275) (width 0.3) (layer F.Cu) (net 19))
 (segment (start 137.2 107.793998) (end 140.718998 104.275) (width 0.3) (layer F.Cu) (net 19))
 (segment (start 137.2 108.925) (end 137.2 107.793998) (width 0.3) (layer F.Cu) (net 19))
 (segment (start 137.625 62.725) (end 137.85 62.95) (width 0.3) (layer F.Cu) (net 2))
 (segment (start 135.5 62.725) (end 137.625 62.725) (width 0.3) (layer F.Cu) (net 2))
 (segment (start 143.32501 63.77501) (end 142.175 62.625) (width 0.3) (layer F.Cu) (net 2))
 (segment (start 143.32501 70.07499) (end 143.32501 63.77501) (width 0.3) (layer F.Cu) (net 2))
 (segment (start 143.3 70.1) (end 143.32501 70.07499) (width 0.3) (layer F.Cu) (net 2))
 (segment (start 141.85 62.95) (end 142.175 62.625) (width 0.3) (layer F.Cu) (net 2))
 (segment (start 137.85 62.95) (end 141.85 62.95) (width 0.3) (layer F.Cu) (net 2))
 (segment (start 135.575 92.9) (end 136.575 93.9) (width 0.3) (layer F.Cu) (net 2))
 (segment (start 135.575 88.7) (end 135.575 92.9) (width 0.3) (layer F.Cu) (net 2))
 (segment (start 137.515 88.7) (end 137.8 88.415) (width 0.3) (layer F.Cu) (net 2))
 (segment (start 135.575 88.7) (end 137.515 88.7) (width 0.3) (layer F.Cu) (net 2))
 (segment (start 142.025 90.525) (end 143.275 91.775) (width 0.3) (layer F.Cu) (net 2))
 (segment (start 142.025 88.075) (end 142.025 90.525) (width 0.3) (layer F.Cu) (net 2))
 (segment (start 137.815 65.525) (end 137.85 65.49) (width 0.3) (layer F.Cu) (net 3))
 (segment (start 135.5 65.525) (end 137.815 65.525) (width 0.3) (layer F.Cu) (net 3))
 (segment (start 140.5 67.65) (end 142.175 65.975) (width 0.3) (layer F.Cu) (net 3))
 (segment (start 140.5 70.1) (end 140.5 67.65) (width 0.3) (layer F.Cu) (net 3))
 (segment (start 140.01 67.65) (end 140.5 67.65) (width 0.3) (layer F.Cu) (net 3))
 (segment (start 137.85 65.49) (end 140.01 67.65) (width 0.3) (layer F.Cu) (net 3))
 (segment (start 135.6 85.875) (end 135.575 85.9) (width 0.3) (layer F.Cu) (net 1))
 (segment (start 137.8 85.875) (end 135.6 85.875) (width 0.3) (layer F.Cu) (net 1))
 (segment (start 140.875 85.875) (end 142.025 84.725) (width 0.3) (layer F.Cu) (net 1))
 (segment (start 137.8 85.875) (end 140.875 85.875) (width 0.3) (layer F.Cu) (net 1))
 (segment (start 138.99 152.75) (end 136.85 150.61) (width 0.3) (layer F.Cu) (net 6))
 (segment (start 140.825 152.75) (end 138.99 152.75) (width 0.3) (layer F.Cu) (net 6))
 (segment (start 135.22499 106.17501) (end 137.125 104.275) (width 0.3) (layer F.Cu) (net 7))
 (segment (start 135.22499 145.06499) (end 135.22499 106.17501) (width 0.3) (layer F.Cu) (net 7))
 (segment (start 136.85 146.69) (end 135.22499 145.06499) (width 0.3) (layer F.Cu) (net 7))
 (segment (start 137.125 101.775) (end 137.125 104.275) (width 0.3) (layer F.Cu) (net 7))
 (segment (start 138.115 144.614722) (end 138.115 142.68) (width 0.3) (layer F.Cu) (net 10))
 (segment (start 140.314279 146.814001) (end 138.115 144.614722) (width 0.3) (layer F.Cu) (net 10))
 (segment (start 140.963723 146.814001) (end 140.314279 146.814001) (width 0.3) (layer F.Cu) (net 10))
 (segment (start 141.889001 147.739279) (end 140.963723 146.814001) (width 0.3) (layer F.Cu) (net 10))
 (segment (start 141.889001 154.390765) (end 141.889001 147.739279) (width 0.3) (layer F.Cu) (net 10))
 (segment (start 140.459766 155.82) (end 141.889001 154.390765) (width 0.3) (layer F.Cu) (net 10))
 (segment (start 138.115 155.82) (end 140.459766 155.82) (width 0.3) (layer F.Cu) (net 10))
 (segment (start 137.95 96.775) (end 136.575 95.4) (width 0.3) (layer F.Cu) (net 20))
 (segment (start 139.625 96.775) (end 137.95 96.775) (width 0.3) (layer F.Cu) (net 20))
 (segment (start 139.625 137.7) (end 139.625 140.425) (width 0.3) (layer F.Cu) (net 5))
 (segment (start 140.825 141.625) (end 140.825 145.75) (width 0.3) (layer F.Cu) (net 5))
 (segment (start 139.625 140.425) (end 140.825 141.625) (width 0.3) (layer F.Cu) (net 5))
 (segment (start 142.975 122.9625) (end 142.3125 123.625) (width 0.3) (layer F.Cu) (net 5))
 (segment (start 142.975 117.4) (end 142.975 122.9625) (width 0.3) (layer F.Cu) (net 5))
 (segment (start 142.3125 135.0125) (end 142.3125 123.625) (width 0.3) (layer F.Cu) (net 5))
 (segment (start 139.625 137.7) (end 142.3125 135.0125) (width 0.3) (layer F.Cu) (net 5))
 (segment (start 142.975 114.25) (end 142.85 114.125) (width 0.3) (layer F.Cu) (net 5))
 (segment (start 142.975 117.4) (end 142.975 114.25) (width 0.3) (layer F.Cu) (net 5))
 (segment (start 136.25 113.225) (end 136.925 113.9) (width 0.3) (layer F.Cu) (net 5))
 (segment (start 136.25 111.025) (end 136.25 113.225) (width 0.3) (layer F.Cu) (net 5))
 (segment (start 136.925 110.669998) (end 136.925 113.9) (width 0.3) (layer F.Cu) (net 5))
 (segment (start 137.569999 110.024999) (end 136.925 110.669998) (width 0.3) (layer F.Cu) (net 5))
 (segment (start 138.749999 110.024999) (end 137.569999 110.024999) (width 0.3) (layer F.Cu) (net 5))
 (segment (start 142.85 114.125) (end 138.749999 110.024999) (width 0.3) (layer F.Cu) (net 5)))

